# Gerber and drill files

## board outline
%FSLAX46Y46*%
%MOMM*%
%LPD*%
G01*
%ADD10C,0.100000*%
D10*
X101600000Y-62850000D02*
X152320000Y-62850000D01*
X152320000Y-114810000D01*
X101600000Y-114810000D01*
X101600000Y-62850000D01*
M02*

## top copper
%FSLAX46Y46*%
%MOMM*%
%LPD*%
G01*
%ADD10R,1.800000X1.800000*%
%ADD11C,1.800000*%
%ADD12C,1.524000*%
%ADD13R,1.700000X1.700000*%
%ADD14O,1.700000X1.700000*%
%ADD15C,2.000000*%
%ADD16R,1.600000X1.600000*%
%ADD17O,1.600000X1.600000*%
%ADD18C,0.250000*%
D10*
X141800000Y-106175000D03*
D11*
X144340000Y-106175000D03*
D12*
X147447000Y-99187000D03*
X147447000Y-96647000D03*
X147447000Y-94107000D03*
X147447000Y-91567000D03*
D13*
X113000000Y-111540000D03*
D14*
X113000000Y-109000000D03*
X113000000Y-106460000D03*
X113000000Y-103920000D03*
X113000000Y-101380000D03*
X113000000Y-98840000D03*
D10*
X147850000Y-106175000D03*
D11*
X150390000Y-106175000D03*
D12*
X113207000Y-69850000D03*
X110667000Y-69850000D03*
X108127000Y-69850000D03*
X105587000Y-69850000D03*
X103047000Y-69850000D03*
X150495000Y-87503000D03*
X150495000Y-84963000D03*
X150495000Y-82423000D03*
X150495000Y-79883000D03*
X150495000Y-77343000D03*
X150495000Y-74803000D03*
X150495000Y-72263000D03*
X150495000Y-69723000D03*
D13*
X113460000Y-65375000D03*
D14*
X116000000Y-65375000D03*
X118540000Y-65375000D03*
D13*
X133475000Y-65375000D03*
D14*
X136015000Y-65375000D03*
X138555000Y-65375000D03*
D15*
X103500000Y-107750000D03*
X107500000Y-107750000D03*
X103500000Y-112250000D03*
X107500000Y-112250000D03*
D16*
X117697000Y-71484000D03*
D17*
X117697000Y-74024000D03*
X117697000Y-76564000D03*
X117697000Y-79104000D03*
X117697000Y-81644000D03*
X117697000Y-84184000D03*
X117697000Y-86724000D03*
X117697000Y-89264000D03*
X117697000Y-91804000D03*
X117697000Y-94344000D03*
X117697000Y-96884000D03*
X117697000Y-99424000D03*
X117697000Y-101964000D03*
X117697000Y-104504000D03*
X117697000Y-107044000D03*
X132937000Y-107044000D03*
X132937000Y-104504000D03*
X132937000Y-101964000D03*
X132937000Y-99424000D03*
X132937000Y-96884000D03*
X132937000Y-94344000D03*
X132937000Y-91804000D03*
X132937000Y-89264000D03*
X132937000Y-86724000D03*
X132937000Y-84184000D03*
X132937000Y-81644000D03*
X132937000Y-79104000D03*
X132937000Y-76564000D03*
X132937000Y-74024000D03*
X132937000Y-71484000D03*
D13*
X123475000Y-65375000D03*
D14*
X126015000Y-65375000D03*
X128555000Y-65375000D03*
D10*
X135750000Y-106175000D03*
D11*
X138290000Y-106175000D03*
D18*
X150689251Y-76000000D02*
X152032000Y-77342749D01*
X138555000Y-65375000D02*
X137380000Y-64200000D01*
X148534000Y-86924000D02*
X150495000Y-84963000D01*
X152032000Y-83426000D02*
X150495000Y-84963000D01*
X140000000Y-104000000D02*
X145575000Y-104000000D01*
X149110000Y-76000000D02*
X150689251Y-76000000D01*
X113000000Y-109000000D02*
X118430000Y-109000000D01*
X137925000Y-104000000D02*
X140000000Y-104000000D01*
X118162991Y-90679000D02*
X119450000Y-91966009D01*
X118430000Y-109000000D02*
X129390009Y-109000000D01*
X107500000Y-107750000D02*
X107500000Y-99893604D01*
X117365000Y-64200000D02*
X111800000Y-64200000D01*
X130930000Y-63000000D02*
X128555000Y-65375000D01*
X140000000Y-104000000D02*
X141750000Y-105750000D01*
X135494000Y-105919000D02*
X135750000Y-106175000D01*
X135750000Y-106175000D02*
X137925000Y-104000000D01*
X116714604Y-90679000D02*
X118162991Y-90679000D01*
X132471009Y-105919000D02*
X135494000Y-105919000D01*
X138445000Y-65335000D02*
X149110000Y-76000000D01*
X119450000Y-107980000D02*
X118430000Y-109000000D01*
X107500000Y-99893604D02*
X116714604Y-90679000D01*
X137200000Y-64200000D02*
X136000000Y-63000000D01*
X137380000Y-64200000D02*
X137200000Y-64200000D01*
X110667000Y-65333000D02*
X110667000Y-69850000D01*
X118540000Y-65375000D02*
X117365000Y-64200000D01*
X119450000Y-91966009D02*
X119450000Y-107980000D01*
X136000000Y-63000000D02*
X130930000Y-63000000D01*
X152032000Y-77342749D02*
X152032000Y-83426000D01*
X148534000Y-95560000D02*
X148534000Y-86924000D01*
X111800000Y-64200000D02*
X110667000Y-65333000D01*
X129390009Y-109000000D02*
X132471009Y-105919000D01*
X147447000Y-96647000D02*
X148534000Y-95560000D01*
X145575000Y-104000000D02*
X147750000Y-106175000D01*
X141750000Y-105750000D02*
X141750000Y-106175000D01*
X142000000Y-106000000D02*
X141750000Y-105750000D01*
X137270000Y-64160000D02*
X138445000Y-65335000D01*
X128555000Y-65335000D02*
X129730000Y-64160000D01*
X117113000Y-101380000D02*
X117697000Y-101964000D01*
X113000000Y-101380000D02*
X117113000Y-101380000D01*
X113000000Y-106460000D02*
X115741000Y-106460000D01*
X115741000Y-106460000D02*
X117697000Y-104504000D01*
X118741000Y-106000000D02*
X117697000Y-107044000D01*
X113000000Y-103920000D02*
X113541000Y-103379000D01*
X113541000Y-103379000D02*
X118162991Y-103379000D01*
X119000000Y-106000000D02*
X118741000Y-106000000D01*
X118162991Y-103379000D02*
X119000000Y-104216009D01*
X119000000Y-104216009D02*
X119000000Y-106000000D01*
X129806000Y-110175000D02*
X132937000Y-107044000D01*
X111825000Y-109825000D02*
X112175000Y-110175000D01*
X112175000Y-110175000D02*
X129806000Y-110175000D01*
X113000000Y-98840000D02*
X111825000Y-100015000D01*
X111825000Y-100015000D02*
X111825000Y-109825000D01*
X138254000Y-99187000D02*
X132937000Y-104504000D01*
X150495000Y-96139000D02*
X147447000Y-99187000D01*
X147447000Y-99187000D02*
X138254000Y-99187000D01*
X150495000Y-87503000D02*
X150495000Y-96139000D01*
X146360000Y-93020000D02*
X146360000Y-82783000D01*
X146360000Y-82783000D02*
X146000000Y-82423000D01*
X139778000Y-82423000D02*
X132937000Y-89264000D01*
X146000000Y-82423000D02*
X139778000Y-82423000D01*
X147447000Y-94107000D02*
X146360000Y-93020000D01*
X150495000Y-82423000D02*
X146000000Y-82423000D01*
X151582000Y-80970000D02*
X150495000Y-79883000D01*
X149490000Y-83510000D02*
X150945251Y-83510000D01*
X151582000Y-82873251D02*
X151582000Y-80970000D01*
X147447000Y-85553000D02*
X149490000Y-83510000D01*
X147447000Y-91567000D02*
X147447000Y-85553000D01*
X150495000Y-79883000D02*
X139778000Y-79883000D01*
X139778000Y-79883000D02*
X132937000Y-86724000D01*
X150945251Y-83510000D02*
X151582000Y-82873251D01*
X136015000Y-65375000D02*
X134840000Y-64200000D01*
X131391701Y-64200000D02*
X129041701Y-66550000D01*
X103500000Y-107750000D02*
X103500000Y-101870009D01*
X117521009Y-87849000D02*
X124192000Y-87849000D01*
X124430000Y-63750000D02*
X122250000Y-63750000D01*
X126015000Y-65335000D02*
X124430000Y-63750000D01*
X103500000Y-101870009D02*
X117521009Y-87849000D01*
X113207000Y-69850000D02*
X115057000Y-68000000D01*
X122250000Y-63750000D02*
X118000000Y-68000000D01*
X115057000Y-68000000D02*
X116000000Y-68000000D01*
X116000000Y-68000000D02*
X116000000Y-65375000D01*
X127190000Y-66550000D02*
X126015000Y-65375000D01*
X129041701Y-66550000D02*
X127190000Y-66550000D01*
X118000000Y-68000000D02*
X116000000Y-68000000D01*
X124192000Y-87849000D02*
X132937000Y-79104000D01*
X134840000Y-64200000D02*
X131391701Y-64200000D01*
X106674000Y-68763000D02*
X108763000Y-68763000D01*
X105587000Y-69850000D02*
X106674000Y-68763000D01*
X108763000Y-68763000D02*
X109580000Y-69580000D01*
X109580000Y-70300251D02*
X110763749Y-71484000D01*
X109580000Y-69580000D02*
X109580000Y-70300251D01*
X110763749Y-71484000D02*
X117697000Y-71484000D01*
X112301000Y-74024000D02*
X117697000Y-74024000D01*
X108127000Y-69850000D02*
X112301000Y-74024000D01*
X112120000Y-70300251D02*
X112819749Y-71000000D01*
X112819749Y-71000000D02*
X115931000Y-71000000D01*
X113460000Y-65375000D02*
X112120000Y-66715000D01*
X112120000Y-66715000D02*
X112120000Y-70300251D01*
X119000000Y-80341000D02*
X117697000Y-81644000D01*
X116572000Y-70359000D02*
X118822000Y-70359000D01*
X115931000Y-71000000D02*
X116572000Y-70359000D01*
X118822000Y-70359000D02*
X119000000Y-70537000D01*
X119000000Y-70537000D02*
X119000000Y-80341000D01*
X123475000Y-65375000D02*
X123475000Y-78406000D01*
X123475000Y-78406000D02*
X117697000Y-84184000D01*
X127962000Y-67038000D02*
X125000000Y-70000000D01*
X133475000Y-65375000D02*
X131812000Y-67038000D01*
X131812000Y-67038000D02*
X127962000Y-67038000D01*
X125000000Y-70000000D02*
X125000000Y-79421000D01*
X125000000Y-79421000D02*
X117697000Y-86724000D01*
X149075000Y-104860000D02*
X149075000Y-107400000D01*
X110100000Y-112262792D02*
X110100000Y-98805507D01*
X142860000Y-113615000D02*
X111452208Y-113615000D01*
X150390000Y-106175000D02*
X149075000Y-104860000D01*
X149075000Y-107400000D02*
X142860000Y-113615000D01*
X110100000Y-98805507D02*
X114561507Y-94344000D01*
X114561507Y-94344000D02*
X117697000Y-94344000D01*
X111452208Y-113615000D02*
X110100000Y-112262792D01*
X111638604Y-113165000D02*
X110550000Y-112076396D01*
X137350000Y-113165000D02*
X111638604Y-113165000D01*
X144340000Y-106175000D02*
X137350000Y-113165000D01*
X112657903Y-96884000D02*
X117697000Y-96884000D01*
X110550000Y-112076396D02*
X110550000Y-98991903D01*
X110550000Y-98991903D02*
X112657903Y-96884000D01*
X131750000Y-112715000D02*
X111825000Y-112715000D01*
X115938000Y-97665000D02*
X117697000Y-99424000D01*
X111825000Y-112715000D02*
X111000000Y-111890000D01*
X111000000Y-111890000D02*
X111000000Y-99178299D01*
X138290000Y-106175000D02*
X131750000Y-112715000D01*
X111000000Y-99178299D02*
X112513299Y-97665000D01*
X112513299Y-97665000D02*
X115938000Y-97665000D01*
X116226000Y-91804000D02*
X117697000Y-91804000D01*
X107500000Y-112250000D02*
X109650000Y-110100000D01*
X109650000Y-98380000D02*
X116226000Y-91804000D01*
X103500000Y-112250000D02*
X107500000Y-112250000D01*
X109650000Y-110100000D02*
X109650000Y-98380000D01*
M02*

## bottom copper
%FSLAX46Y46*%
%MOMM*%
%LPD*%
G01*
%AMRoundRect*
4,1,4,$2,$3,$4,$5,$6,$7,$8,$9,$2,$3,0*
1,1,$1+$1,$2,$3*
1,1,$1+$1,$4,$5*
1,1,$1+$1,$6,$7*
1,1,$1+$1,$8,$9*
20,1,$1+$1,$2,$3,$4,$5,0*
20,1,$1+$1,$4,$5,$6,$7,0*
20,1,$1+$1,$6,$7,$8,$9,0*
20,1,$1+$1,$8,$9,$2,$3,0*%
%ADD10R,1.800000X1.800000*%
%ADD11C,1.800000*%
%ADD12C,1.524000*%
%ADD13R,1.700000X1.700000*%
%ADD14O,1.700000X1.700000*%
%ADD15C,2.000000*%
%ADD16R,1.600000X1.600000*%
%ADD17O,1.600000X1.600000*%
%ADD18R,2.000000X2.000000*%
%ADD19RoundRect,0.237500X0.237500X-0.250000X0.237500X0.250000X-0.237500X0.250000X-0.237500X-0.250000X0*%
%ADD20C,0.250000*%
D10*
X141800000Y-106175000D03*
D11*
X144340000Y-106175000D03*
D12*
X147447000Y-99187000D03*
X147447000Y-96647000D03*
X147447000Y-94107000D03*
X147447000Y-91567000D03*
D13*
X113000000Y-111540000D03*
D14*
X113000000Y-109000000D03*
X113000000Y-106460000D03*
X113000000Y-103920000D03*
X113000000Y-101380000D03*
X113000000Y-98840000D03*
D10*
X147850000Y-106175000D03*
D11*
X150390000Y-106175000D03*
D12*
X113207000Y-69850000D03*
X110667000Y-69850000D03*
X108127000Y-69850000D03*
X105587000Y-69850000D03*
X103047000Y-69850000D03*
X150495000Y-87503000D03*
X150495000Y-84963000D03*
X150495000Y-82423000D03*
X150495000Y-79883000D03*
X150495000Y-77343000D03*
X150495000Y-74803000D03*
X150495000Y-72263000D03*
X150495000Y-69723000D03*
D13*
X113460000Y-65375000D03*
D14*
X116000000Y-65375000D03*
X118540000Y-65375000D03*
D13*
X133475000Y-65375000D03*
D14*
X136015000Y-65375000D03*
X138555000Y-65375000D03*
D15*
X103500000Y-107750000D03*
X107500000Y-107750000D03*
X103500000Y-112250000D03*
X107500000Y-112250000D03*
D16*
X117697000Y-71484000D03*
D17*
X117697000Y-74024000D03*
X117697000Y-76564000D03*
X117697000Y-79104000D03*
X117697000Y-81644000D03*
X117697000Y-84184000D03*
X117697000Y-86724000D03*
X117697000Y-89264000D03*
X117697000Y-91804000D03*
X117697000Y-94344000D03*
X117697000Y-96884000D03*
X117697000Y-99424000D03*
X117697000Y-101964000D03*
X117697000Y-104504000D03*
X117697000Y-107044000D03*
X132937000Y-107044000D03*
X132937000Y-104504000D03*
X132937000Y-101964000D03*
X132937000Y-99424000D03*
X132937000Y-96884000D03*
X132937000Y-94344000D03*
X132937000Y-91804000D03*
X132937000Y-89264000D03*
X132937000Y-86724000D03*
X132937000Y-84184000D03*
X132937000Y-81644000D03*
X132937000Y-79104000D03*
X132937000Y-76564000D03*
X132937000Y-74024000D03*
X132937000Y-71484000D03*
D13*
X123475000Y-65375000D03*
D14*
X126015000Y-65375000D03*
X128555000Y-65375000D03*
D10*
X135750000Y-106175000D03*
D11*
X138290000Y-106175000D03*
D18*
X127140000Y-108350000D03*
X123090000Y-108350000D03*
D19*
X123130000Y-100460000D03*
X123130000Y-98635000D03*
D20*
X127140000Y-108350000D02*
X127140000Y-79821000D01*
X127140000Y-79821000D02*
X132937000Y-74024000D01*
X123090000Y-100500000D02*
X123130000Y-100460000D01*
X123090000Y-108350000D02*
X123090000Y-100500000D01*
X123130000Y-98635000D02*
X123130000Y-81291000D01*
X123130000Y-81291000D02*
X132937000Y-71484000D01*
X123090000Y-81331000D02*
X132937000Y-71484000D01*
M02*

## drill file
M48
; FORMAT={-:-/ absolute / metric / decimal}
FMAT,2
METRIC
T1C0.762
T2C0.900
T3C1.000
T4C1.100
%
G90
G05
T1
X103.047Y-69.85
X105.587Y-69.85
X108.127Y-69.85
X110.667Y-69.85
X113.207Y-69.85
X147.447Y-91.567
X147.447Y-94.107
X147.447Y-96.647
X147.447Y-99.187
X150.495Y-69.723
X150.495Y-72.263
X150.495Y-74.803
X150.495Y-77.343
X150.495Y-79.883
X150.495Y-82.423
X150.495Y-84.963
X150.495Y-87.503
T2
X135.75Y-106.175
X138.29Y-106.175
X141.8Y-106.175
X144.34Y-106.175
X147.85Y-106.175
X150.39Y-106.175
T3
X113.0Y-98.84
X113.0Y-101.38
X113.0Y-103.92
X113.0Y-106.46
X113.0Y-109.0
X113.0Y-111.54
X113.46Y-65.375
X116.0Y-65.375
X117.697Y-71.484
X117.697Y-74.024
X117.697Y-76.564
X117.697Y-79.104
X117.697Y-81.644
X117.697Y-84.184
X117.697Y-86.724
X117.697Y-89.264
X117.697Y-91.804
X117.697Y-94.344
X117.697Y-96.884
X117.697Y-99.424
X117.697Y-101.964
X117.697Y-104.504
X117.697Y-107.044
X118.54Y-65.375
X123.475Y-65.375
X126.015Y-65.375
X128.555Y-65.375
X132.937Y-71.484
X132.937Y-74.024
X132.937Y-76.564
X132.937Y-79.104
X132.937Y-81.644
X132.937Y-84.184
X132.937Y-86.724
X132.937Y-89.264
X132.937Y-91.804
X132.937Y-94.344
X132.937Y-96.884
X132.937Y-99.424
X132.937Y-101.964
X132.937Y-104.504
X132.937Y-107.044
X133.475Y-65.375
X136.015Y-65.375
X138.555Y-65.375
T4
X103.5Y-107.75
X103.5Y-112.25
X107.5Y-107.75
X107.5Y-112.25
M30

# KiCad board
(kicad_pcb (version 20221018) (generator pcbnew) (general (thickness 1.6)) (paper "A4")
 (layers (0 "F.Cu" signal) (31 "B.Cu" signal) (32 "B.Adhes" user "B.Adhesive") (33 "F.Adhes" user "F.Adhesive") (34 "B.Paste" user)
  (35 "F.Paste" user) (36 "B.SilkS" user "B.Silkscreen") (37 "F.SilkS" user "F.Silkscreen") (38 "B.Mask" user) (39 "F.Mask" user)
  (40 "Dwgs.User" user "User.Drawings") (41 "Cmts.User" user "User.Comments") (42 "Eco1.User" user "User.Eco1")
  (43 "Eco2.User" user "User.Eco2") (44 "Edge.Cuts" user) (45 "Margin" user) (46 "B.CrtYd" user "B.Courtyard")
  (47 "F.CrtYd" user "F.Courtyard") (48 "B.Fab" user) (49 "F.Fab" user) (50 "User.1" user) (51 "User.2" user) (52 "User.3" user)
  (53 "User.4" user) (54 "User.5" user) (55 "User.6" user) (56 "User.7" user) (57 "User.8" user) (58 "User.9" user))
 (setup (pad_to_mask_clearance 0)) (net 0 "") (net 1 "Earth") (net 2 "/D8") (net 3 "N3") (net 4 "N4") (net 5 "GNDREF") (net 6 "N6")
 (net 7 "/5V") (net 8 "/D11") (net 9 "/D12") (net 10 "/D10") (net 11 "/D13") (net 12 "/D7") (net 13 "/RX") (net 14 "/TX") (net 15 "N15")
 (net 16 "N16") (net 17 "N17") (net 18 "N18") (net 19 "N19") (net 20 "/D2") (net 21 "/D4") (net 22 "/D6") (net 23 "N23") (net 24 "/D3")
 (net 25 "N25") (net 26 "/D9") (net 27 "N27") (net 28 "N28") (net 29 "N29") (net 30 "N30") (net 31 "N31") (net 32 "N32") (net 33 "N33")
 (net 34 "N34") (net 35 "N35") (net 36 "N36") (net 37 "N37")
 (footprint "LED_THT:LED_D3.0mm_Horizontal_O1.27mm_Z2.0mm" (layer "F.Cu") (at 141.8 106.175)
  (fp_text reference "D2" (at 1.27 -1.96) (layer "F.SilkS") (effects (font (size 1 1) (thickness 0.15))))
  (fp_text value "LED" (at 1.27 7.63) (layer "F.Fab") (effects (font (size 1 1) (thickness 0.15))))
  (pad "1" thru_hole rect (at 0 0) (size 1.8 1.8) (drill 0.9) (layers "*.Cu" "*.Mask") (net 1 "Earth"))
  (pad "2" thru_hole circle (at 2.54 0) (size 1.8 1.8) (drill 0.9) (layers "*.Cu" "*.Mask") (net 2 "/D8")))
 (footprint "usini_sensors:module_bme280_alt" (layer "F.Cu") (at 147.447 91.567 180)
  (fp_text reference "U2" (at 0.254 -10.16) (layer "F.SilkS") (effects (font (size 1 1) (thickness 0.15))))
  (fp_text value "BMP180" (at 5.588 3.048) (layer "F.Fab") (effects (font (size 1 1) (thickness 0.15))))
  (pad "1" thru_hole circle (at 0 -7.62 180) (size 1.524 1.524) (drill 0.762) (layers "*.Cu" "*.Mask") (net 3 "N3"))
  (pad "2" thru_hole circle (at 0 -5.08 180) (size 1.524 1.524) (drill 0.762) (layers "*.Cu" "*.Mask") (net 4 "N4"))
  (pad "3" thru_hole circle (at 0 -2.54 180) (size 1.524 1.524) (drill 0.762) (layers "*.Cu" "*.Mask") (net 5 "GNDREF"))
  (pad "4" thru_hole circle (at 0 0 180) (size 1.524 1.524) (drill 0.762) (layers "*.Cu" "*.Mask") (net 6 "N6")))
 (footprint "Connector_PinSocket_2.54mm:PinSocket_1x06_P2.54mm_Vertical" (layer "F.Cu") (at 113 111.54 180)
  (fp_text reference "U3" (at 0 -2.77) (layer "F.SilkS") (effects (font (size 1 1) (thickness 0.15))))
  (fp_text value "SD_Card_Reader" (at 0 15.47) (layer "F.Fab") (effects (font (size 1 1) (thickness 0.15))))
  (pad "1" thru_hole rect (at 0 0 180) (size 1.7 1.7) (drill 1) (layers "*.Cu" "*.Mask") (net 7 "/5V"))
  (pad "2" thru_hole oval (at 0 2.54 180) (size 1.7 1.7) (drill 1) (layers "*.Cu" "*.Mask") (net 1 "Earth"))
  (pad "3" thru_hole oval (at 0 5.08 180) (size 1.7 1.7) (drill 1) (layers "*.Cu" "*.Mask") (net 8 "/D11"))
  (pad "4" thru_hole oval (at 0 7.62 180) (size 1.7 1.7) (drill 1) (layers "*.Cu" "*.Mask") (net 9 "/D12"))
  (pad "5" thru_hole oval (at 0 10.16 180) (size 1.7 1.7) (drill 1) (layers "*.Cu" "*.Mask") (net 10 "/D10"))
  (pad "6" thru_hole oval (at 0 12.7 180) (size 1.7 1.7) (drill 1) (layers "*.Cu" "*.Mask") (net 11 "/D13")))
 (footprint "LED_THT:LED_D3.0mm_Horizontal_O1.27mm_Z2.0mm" (layer "F.Cu") (at 147.85 106.175)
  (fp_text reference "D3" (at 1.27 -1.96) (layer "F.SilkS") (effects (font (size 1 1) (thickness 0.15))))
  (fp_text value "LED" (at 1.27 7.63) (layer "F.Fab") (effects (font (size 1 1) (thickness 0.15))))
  (pad "1" thru_hole rect (at 0 0) (size 1.8 1.8) (drill 0.9) (layers "*.Cu" "*.Mask") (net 1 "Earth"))
  (pad "2" thru_hole circle (at 2.54 0) (size 1.8 1.8) (drill 0.9) (layers "*.Cu" "*.Mask") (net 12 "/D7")))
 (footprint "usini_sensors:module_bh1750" (layer "F.Cu") (at 103.047 69.85 -90)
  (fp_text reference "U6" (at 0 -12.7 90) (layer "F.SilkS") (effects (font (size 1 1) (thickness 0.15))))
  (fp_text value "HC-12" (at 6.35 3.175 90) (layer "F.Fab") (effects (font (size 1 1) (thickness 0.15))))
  (pad "1" thru_hole circle (at 0 -10.16 270) (size 1.524 1.524) (drill 0.762) (layers "*.Cu" "*.Mask") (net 6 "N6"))
  (pad "2" thru_hole circle (at 0 -7.62 270) (size 1.524 1.524) (drill 0.762) (layers "*.Cu" "*.Mask") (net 5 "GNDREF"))
  (pad "3" thru_hole circle (at 0 -5.08 270) (size 1.524 1.524) (drill 0.762) (layers "*.Cu" "*.Mask") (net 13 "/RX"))
  (pad "4" thru_hole circle (at 0 -2.54 270) (size 1.524 1.524) (drill 0.762) (layers "*.Cu" "*.Mask") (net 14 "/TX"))
  (pad "5" thru_hole circle (at 0 0 270) (size 1.524 1.524) (drill 0.762) (layers "*.Cu" "*.Mask") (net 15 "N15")))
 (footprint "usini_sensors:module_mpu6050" (layer "F.Cu") (at 150.495 69.723 180)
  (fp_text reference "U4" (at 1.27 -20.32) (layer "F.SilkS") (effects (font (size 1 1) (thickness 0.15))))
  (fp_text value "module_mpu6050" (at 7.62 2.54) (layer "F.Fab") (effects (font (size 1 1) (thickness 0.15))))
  (pad "1" thru_hole circle (at 0 -17.78 180) (size 1.524 1.524) (drill 0.762) (layers "*.Cu" "*.Mask") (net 6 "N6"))
  (pad "2" thru_hole circle (at 0 -15.24 180) (size 1.524 1.524) (drill 0.762) (layers "*.Cu" "*.Mask") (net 5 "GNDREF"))
  (pad "3" thru_hole circle (at 0 -12.7 180) (size 1.524 1.524) (drill 0.762) (layers "*.Cu" "*.Mask") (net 4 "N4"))
  (pad "4" thru_hole circle (at 0 -10.16 180) (size 1.524 1.524) (drill 0.762) (layers "*.Cu" "*.Mask") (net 3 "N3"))
  (pad "5" thru_hole circle (at 0 -7.62 180) (size 1.524 1.524) (drill 0.762) (layers "*.Cu" "*.Mask") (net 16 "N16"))
  (pad "6" thru_hole circle (at 0 -5.08 180) (size 1.524 1.524) (drill 0.762) (layers "*.Cu" "*.Mask") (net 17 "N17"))
  (pad "7" thru_hole circle (at 0 -2.54 180) (size 1.524 1.524) (drill 0.762) (layers "*.Cu" "*.Mask") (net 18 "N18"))
  (pad "8" thru_hole circle (at 0 0 180) (size 1.524 1.524) (drill 0.762) (layers "*.Cu" "*.Mask") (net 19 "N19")))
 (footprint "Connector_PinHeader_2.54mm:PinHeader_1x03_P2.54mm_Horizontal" (layer "F.Cu") (at 113.46 65.375 90)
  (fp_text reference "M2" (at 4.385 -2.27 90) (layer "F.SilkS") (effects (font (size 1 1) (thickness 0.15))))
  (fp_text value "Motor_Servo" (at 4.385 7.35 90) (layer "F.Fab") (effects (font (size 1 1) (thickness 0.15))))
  (pad "1" thru_hole rect (at 0 0 90) (size 1.7 1.7) (drill 1) (layers "*.Cu" "*.Mask") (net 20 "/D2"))
  (pad "2" thru_hole oval (at 0 2.54 90) (size 1.7 1.7) (drill 1) (layers "*.Cu" "*.Mask") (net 7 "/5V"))
  (pad "3" thru_hole oval (at 0 5.08 90) (size 1.7 1.7) (drill 1) (layers "*.Cu" "*.Mask") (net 1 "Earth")))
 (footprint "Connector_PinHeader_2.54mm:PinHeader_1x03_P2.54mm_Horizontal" (layer "F.Cu") (at 133.475 65.375 90)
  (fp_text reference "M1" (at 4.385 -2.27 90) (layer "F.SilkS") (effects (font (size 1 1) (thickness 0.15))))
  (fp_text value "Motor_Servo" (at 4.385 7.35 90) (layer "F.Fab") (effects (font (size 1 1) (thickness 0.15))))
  (pad "1" thru_hole rect (at 0 0 90) (size 1.7 1.7) (drill 1) (layers "*.Cu" "*.Mask") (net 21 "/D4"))
  (pad "2" thru_hole oval (at 0 2.54 90) (size 1.7 1.7) (drill 1) (layers "*.Cu" "*.Mask") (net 7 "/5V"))
  (pad "3" thru_hole oval (at 0 5.08 90) (size 1.7 1.7) (drill 1) (layers "*.Cu" "*.Mask") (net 1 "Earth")))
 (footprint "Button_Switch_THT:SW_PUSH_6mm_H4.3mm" (layer "F.Cu") (at 101 107.75)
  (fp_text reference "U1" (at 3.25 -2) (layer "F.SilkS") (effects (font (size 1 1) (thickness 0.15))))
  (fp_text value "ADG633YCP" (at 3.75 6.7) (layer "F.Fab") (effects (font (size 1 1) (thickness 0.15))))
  (pad "1" thru_hole circle (at 2.5 0 90) (size 2 2) (drill 1.1) (layers "*.Cu" "*.Mask") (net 7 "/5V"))
  (pad "1" thru_hole circle (at 6.5 0 90) (size 2 2) (drill 1.1) (layers "*.Cu" "*.Mask") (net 7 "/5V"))
  (pad "2" thru_hole circle (at 2.5 4.5 90) (size 2 2) (drill 1.1) (layers "*.Cu" "*.Mask") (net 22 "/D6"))
  (pad "2" thru_hole circle (at 6.5 4.5 90) (size 2 2) (drill 1.1) (layers "*.Cu" "*.Mask") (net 22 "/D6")))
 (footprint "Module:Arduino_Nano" (layer "F.Cu") (at 117.697 71.484)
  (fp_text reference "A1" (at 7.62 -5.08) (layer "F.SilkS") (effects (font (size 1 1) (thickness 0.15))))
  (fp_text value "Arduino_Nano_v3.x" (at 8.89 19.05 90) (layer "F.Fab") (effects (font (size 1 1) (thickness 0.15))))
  (pad "1" thru_hole rect (at 0 0) (size 1.6 1.6) (drill 1) (layers "*.Cu" "*.Mask") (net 14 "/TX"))
  (pad "2" thru_hole oval (at 0 2.54) (size 1.6 1.6) (drill 1) (layers "*.Cu" "*.Mask") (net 13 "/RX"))
  (pad "3" thru_hole oval (at 0 5.08) (size 1.6 1.6) (drill 1) (layers "*.Cu" "*.Mask") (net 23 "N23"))
  (pad "4" thru_hole oval (at 0 7.62) (size 1.6 1.6) (drill 1) (layers "*.Cu" "*.Mask") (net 1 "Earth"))
  (pad "5" thru_hole oval (at 0 10.16) (size 1.6 1.6) (drill 1) (layers "*.Cu" "*.Mask") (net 20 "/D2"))
  (pad "6" thru_hole oval (at 0 12.7) (size 1.6 1.6) (drill 1) (layers "*.Cu" "*.Mask") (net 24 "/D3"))
  (pad "7" thru_hole oval (at 0 15.24) (size 1.6 1.6) (drill 1) (layers "*.Cu" "*.Mask") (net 21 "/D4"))
  (pad "8" thru_hole oval (at 0 17.78) (size 1.6 1.6) (drill 1) (layers "*.Cu" "*.Mask") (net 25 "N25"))
  (pad "9" thru_hole oval (at 0 20.32) (size 1.6 1.6) (drill 1) (layers "*.Cu" "*.Mask") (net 22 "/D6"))
  (pad "10" thru_hole oval (at 0 22.86) (size 1.6 1.6) (drill 1) (layers "*.Cu" "*.Mask") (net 12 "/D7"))
  (pad "11" thru_hole oval (at 0 25.4) (size 1.6 1.6) (drill 1) (layers "*.Cu" "*.Mask") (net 2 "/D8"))
  (pad "12" thru_hole oval (at 0 27.94) (size 1.6 1.6) (drill 1) (layers "*.Cu" "*.Mask") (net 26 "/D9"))
  (pad "13" thru_hole oval (at 0 30.48) (size 1.6 1.6) (drill 1) (layers "*.Cu" "*.Mask") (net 10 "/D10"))
  (pad "14" thru_hole oval (at 0 33.02) (size 1.6 1.6) (drill 1) (layers "*.Cu" "*.Mask") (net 8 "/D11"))
  (pad "15" thru_hole oval (at 0 35.56) (size 1.6 1.6) (drill 1) (layers "*.Cu" "*.Mask") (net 9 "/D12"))
  (pad "16" thru_hole oval (at 15.24 35.56) (size 1.6 1.6) (drill 1) (layers "*.Cu" "*.Mask") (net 11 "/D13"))
  (pad "17" thru_hole oval (at 15.24 33.02) (size 1.6 1.6) (drill 1) (layers "*.Cu" "*.Mask") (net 6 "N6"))
  (pad "18" thru_hole oval (at 15.24 30.48) (size 1.6 1.6) (drill 1) (layers "*.Cu" "*.Mask") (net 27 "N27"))
  (pad "19" thru_hole oval (at 15.24 27.94) (size 1.6 1.6) (drill 1) (layers "*.Cu" "*.Mask") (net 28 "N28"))
  (pad "20" thru_hole oval (at 15.24 25.4) (size 1.6 1.6) (drill 1) (layers "*.Cu" "*.Mask") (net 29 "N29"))
  (pad "21" thru_hole oval (at 15.24 22.86) (size 1.6 1.6) (drill 1) (layers "*.Cu" "*.Mask") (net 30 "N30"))
  (pad "22" thru_hole oval (at 15.24 20.32) (size 1.6 1.6) (drill 1) (layers "*.Cu" "*.Mask") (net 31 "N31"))
  (pad "23" thru_hole oval (at 15.24 17.78) (size 1.6 1.6) (drill 1) (layers "*.Cu" "*.Mask") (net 4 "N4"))
  (pad "24" thru_hole oval (at 15.24 15.24) (size 1.6 1.6) (drill 1) (layers "*.Cu" "*.Mask") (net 3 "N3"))
  (pad "25" thru_hole oval (at 15.24 12.7) (size 1.6 1.6) (drill 1) (layers "*.Cu" "*.Mask") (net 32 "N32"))
  (pad "26" thru_hole oval (at 15.24 10.16) (size 1.6 1.6) (drill 1) (layers "*.Cu" "*.Mask") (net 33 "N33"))
  (pad "27" thru_hole oval (at 15.24 7.62) (size 1.6 1.6) (drill 1) (layers "*.Cu" "*.Mask") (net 7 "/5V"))
  (pad "28" thru_hole oval (at 15.24 5.08) (size 1.6 1.6) (drill 1) (layers "*.Cu" "*.Mask") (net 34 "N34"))
  (pad "29" thru_hole oval (at 15.24 2.54) (size 1.6 1.6) (drill 1) (layers "*.Cu" "*.Mask") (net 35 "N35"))
  (pad "30" thru_hole oval (at 15.24 0) (size 1.6 1.6) (drill 1) (layers "*.Cu" "*.Mask") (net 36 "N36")))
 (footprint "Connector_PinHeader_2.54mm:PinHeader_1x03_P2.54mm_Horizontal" (layer "F.Cu") (at 123.475 65.375 90)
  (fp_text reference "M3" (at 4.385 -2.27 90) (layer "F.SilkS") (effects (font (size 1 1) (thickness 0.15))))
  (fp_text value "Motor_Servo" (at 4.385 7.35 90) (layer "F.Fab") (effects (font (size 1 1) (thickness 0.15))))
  (pad "1" thru_hole rect (at 0 0 90) (size 1.7 1.7) (drill 1) (layers "*.Cu" "*.Mask") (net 24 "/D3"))
  (pad "2" thru_hole oval (at 0 2.54 90) (size 1.7 1.7) (drill 1) (layers "*.Cu" "*.Mask") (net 7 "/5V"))
  (pad "3" thru_hole oval (at 0 5.08 90) (size 1.7 1.7) (drill 1) (layers "*.Cu" "*.Mask") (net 1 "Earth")))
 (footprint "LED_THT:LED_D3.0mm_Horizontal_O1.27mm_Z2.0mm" (layer "F.Cu") (at 135.75 106.175)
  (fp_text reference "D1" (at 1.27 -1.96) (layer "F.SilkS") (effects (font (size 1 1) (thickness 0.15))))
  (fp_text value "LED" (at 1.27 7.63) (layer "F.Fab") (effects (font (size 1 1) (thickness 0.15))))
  (pad "1" thru_hole rect (at 0 0) (size 1.8 1.8) (drill 0.9) (layers "*.Cu" "*.Mask") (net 1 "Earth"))
  (pad "2" thru_hole circle (at 2.54 0) (size 1.8 1.8) (drill 0.9) (layers "*.Cu" "*.Mask") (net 26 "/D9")))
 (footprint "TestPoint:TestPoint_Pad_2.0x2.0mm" (layer "B.Cu") (at 127.14 108.35 -90)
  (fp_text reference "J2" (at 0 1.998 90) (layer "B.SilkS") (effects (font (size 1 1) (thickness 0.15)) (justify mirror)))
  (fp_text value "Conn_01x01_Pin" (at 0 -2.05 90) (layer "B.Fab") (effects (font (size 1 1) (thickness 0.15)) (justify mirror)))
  (pad "1" smd rect (at 0 0 270) (size 2 2) (layers "B.Cu" "B.Mask") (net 35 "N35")))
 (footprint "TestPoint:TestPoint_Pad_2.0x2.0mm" (layer "B.Cu") (at 123.09 108.35 -90)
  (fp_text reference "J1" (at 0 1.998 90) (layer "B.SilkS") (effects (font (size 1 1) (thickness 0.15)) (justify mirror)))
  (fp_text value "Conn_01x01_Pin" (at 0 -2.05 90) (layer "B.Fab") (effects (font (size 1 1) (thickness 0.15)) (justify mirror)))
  (pad "1" smd rect (at 0 0 270) (size 2 2) (layers "B.Cu" "B.Mask") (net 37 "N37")))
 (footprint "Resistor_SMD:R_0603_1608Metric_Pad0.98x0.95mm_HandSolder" (layer "B.Cu") (at 123.13 99.5475 90)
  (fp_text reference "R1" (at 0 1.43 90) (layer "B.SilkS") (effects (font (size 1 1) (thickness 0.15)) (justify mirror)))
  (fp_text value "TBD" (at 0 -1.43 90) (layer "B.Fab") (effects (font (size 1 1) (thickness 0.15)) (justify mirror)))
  (pad "1" smd roundrect (at -0.9125 0 90) (size 0.975 0.95) (layers "B.Cu" "B.Paste" "B.Mask") (roundrect_rratio 0.25) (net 37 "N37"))
  (pad "2" smd roundrect (at 0.9125 0 90) (size 0.975 0.95) (layers "B.Cu" "B.Paste" "B.Mask") (roundrect_rratio 0.25) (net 36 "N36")))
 (gr_rect (start 101.6 62.85) (end 152.32 114.81) (stroke (width 0.1) (type default)) (fill none) (layer "Edge.Cuts"))
 (segment (start 150.689251 76) (end 152.032 77.342749) (width 0.25) (layer "F.Cu") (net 1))
 (segment (start 138.555 65.375) (end 137.38 64.2) (width 0.25) (layer "F.Cu") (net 1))
 (segment (start 148.534 86.924) (end 150.495 84.963) (width 0.25) (layer "F.Cu") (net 1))
 (segment (start 152.032 83.426) (end 150.495 84.963) (width 0.25) (layer "F.Cu") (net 1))
 (segment (start 140 104) (end 145.575 104) (width 0.25) (layer "F.Cu") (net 1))
 (segment (start 149.11 76) (end 150.689251 76) (width 0.25) (layer "F.Cu") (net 1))
 (segment (start 113 109) (end 118.43 109) (width 0.25) (layer "F.Cu") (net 1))
 (segment (start 137.925 104) (end 140 104) (width 0.25) (layer "F.Cu") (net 1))
 (segment (start 118.162991 90.679) (end 119.45 91.966009) (width 0.25) (layer "F.Cu") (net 1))
 (segment (start 118.43 109) (end 129.390009 109) (width 0.25) (layer "F.Cu") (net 1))
 (segment (start 107.5 107.75) (end 107.5 99.893604) (width 0.25) (layer "F.Cu") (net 1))
 (segment (start 117.365 64.2) (end 111.8 64.2) (width 0.25) (layer "F.Cu") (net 1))
 (segment (start 130.93 63) (end 128.555 65.375) (width 0.25) (layer "F.Cu") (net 1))
 (segment (start 140 104) (end 141.75 105.75) (width 0.25) (layer "F.Cu") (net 1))
 (segment (start 135.494 105.919) (end 135.75 106.175) (width 0.25) (layer "F.Cu") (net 1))
 (segment (start 135.75 106.175) (end 137.925 104) (width 0.25) (layer "F.Cu") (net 1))
 (segment (start 116.714604 90.679) (end 118.162991 90.679) (width 0.25) (layer "F.Cu") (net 1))
 (segment (start 132.471009 105.919) (end 135.494 105.919) (width 0.25) (layer "F.Cu") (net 1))
 (segment (start 138.445 65.335) (end 149.11 76) (width 0.25) (layer "F.Cu") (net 1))
 (segment (start 119.45 107.98) (end 118.43 109) (width 0.25) (layer "F.Cu") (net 1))
 (segment (start 107.5 99.893604) (end 116.714604 90.679) (width 0.25) (layer "F.Cu") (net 1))
 (segment (start 137.2 64.2) (end 136 63) (width 0.25) (layer "F.Cu") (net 1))
 (segment (start 137.38 64.2) (end 137.2 64.2) (width 0.25) (layer "F.Cu") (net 1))
 (segment (start 110.667 65.333) (end 110.667 69.85) (width 0.25) (layer "F.Cu") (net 1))
 (segment (start 118.54 65.375) (end 117.365 64.2) (width 0.25) (layer "F.Cu") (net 1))
 (segment (start 119.45 91.966009) (end 119.45 107.98) (width 0.25) (layer "F.Cu") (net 1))
 (segment (start 136 63) (end 130.93 63) (width 0.25) (layer "F.Cu") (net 1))
 (segment (start 152.032 77.342749) (end 152.032 83.426) (width 0.25) (layer "F.Cu") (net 1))
 (segment (start 148.534 95.56) (end 148.534 86.924) (width 0.25) (layer "F.Cu") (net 1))
 (segment (start 111.8 64.2) (end 110.667 65.333) (width 0.25) (layer "F.Cu") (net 1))
 (segment (start 129.390009 109) (end 132.471009 105.919) (width 0.25) (layer "F.Cu") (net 1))
 (segment (start 147.447 96.647) (end 148.534 95.56) (width 0.25) (layer "F.Cu") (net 1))
 (segment (start 145.575 104) (end 147.75 106.175) (width 0.25) (layer "F.Cu") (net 1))
 (segment (start 141.75 105.75) (end 141.75 106.175) (width 0.25) (layer "F.Cu") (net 1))
 (segment (start 142 106) (end 141.75 105.75) (width 0.25) (layer "F.Cu") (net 1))
 (segment (start 137.27 64.16) (end 138.445 65.335) (width 0.25) (layer "F.Cu") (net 1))
 (segment (start 128.555 65.335) (end 129.73 64.16) (width 0.25) (layer "F.Cu") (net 1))
 (segment (start 117.113 101.38) (end 117.697 101.964) (width 0.25) (layer "F.Cu") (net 10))
 (segment (start 113 101.38) (end 117.113 101.38) (width 0.25) (layer "F.Cu") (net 10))
 (segment (start 113 106.46) (end 115.741 106.46) (width 0.25) (layer "F.Cu") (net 8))
 (segment (start 115.741 106.46) (end 117.697 104.504) (width 0.25) (layer "F.Cu") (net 8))
 (segment (start 118.741 106) (end 117.697 107.044) (width 0.25) (layer "F.Cu") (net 9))
 (segment (start 113 103.92) (end 113.541 103.379) (width 0.25) (layer "F.Cu") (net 9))
 (segment (start 113.541 103.379) (end 118.162991 103.379) (width 0.25) (layer "F.Cu") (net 9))
 (segment (start 119 106) (end 118.741 106) (width 0.25) (layer "F.Cu") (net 9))
 (segment (start 118.162991 103.379) (end 119 104.216009) (width 0.25) (layer "F.Cu") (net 9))
 (segment (start 119 104.216009) (end 119 106) (width 0.25) (layer "F.Cu") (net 9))
 (segment (start 129.806 110.175) (end 132.937 107.044) (width 0.25) (layer "F.Cu") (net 11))
 (segment (start 111.825 109.825) (end 112.175 110.175) (width 0.25) (layer "F.Cu") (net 11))
 (segment (start 112.175 110.175) (end 129.806 110.175) (width 0.25) (layer "F.Cu") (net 11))
 (segment (start 113 98.84) (end 111.825 100.015) (width 0.25) (layer "F.Cu") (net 11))
 (segment (start 111.825 100.015) (end 111.825 109.825) (width 0.25) (layer "F.Cu") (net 11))
 (segment (start 138.254 99.187) (end 132.937 104.504) (width 0.25) (layer "F.Cu") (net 6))
 (segment (start 150.495 96.139) (end 147.447 99.187) (width 0.25) (layer "F.Cu") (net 6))
 (segment (start 147.447 99.187) (end 138.254 99.187) (width 0.25) (layer "F.Cu") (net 6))
 (segment (start 150.495 87.503) (end 150.495 96.139) (width 0.25) (layer "F.Cu") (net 6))
 (segment (start 146.36 93.02) (end 146.36 82.783) (width 0.25) (layer "F.Cu") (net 4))
 (segment (start 146.36 82.783) (end 146 82.423) (width 0.25) (layer "F.Cu") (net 4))
 (segment (start 139.778 82.423) (end 132.937 89.264) (width 0.25) (layer "F.Cu") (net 4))
 (segment (start 146 82.423) (end 139.778 82.423) (width 0.25) (layer "F.Cu") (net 4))
 (segment (start 147.447 94.107) (end 146.36 93.02) (width 0.25) (layer "F.Cu") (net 4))
 (segment (start 150.495 82.423) (end 146 82.423) (width 0.25) (layer "F.Cu") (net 4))
 (segment (start 151.582 80.97) (end 150.495 79.883) (width 0.25) (layer "F.Cu") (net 3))
 (segment (start 149.49 83.51) (end 150.945251 83.51) (width 0.25) (layer "F.Cu") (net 3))
 (segment (start 151.582 82.873251) (end 151.582 80.97) (width 0.25) (layer "F.Cu") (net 3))
 (segment (start 147.447 85.553) (end 149.49 83.51) (width 0.25) (layer "F.Cu") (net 3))
 (segment (start 147.447 91.567) (end 147.447 85.553) (width 0.25) (layer "F.Cu") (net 3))
 (segment (start 150.495 79.883) (end 139.778 79.883) (width 0.25) (layer "F.Cu") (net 3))
 (segment (start 139.778 79.883) (end 132.937 86.724) (width 0.25) (layer "F.Cu") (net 3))
 (segment (start 150.945251 83.51) (end 151.582 82.873251) (width 0.25) (layer "F.Cu") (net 3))
 (segment (start 136.015 65.375) (end 134.84 64.2) (width 0.25) (layer "F.Cu") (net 7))
 (segment (start 131.391701 64.2) (end 129.041701 66.55) (width 0.25) (layer "F.Cu") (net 7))
 (segment (start 103.5 107.75) (end 103.5 101.870009) (width 0.25) (layer "F.Cu") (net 7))
 (segment (start 117.521009 87.849) (end 124.192 87.849) (width 0.25) (layer "F.Cu") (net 7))
 (segment (start 124.43 63.75) (end 122.25 63.75) (width 0.25) (layer "F.Cu") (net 7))
 (segment (start 126.015 65.335) (end 124.43 63.75) (width 0.25) (layer "F.Cu") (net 7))
 (segment (start 103.5 101.870009) (end 117.521009 87.849) (width 0.25) (layer "F.Cu") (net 7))
 (segment (start 113.207 69.85) (end 115.057 68) (width 0.25) (layer "F.Cu") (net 7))
 (segment (start 122.25 63.75) (end 118 68) (width 0.25) (layer "F.Cu") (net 7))
 (segment (start 115.057 68) (end 116 68) (width 0.25) (layer "F.Cu") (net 7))
 (segment (start 116 68) (end 116 65.375) (width 0.25) (layer "F.Cu") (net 7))
 (segment (start 127.19 66.55) (end 126.015 65.375) (width 0.25) (layer "F.Cu") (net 7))
 (segment (start 129.041701 66.55) (end 127.19 66.55) (width 0.25) (layer "F.Cu") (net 7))
 (segment (start 118 68) (end 116 68) (width 0.25) (layer "F.Cu") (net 7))
 (segment (start 124.192 87.849) (end 132.937 79.104) (width 0.25) (layer "F.Cu") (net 7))
 (segment (start 134.84 64.2) (end 131.391701 64.2) (width 0.25) (layer "F.Cu") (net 7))
 (segment (start 106.674 68.763) (end 108.763 68.763) (width 0.25) (layer "F.Cu") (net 14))
 (segment (start 105.587 69.85) (end 106.674 68.763) (width 0.25) (layer "F.Cu") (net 14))
 (segment (start 108.763 68.763) (end 109.58 69.58) (width 0.25) (layer "F.Cu") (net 14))
 (segment (start 109.58 70.300251) (end 110.763749 71.484) (width 0.25) (layer "F.Cu") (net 14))
 (segment (start 109.58 69.58) (end 109.58 70.300251) (width 0.25) (layer "F.Cu") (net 14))
 (segment (start 110.763749 71.484) (end 117.697 71.484) (width 0.25) (layer "F.Cu") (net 14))
 (segment (start 112.301 74.024) (end 117.697 74.024) (width 0.25) (layer "F.Cu") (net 13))
 (segment (start 108.127 69.85) (end 112.301 74.024) (width 0.25) (layer "F.Cu") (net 13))
 (segment (start 112.12 70.300251) (end 112.819749 71) (width 0.25) (layer "F.Cu") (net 20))
 (segment (start 112.819749 71) (end 115.931 71) (width 0.25) (layer "F.Cu") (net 20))
 (segment (start 113.46 65.375) (end 112.12 66.715) (width 0.25) (layer "F.Cu") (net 20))
 (segment (start 112.12 66.715) (end 112.12 70.300251) (width 0.25) (layer "F.Cu") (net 20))
 (segment (start 119 80.341) (end 117.697 81.644) (width 0.25) (layer "F.Cu") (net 20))
 (segment (start 116.572 70.359) (end 118.822 70.359) (width 0.25) (layer "F.Cu") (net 20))
 (segment (start 115.931 71) (end 116.572 70.359) (width 0.25) (layer "F.Cu") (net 20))
 (segment (start 118.822 70.359) (end 119 70.537) (width 0.25) (layer "F.Cu") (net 20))
 (segment (start 119 70.537) (end 119 80.341) (width 0.25) (layer "F.Cu") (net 20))
 (segment (start 123.475 65.375) (end 123.475 78.406) (width 0.25) (layer "F.Cu") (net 24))
 (segment (start 123.475 78.406) (end 117.697 84.184) (width 0.25) (layer "F.Cu") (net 24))
 (segment (start 127.962 67.038) (end 125 70) (width 0.25) (layer "F.Cu") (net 21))
 (segment (start 133.475 65.375) (end 131.812 67.038) (width 0.25) (layer "F.Cu") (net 21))
 (segment (start 131.812 67.038) (end 127.962 67.038) (width 0.25) (layer "F.Cu") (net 21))
 (segment (start 125 70) (end 125 79.421) (width 0.25) (layer "F.Cu") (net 21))
 (segment (start 125 79.421) (end 117.697 86.724) (width 0.25) (layer "F.Cu") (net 21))
 (segment (start 149.075 104.86) (end 149.075 107.4) (width 0.25) (layer "F.Cu") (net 12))
 (segment (start 110.1 112.262792) (end 110.1 98.805507) (width 0.25) (layer "F.Cu") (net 12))
 (segment (start 142.86 113.615) (end 111.452208 113.615) (width 0.25) (layer "F.Cu") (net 12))
 (segment (start 150.39 106.175) (end 149.075 104.86) (width 0.25) (layer "F.Cu") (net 12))
 (segment (start 149.075 107.4) (end 142.86 113.615) (width 0.25) (layer "F.Cu") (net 12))
 (segment (start 110.1 98.805507) (end 114.561507 94.344) (width 0.25) (layer "F.Cu") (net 12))
 (segment (start 114.561507 94.344) (end 117.697 94.344) (width 0.25) (layer "F.Cu") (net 12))
 (segment (start 111.452208 113.615) (end 110.1 112.262792) (width 0.25) (layer "F.Cu") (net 12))
 (segment (start 111.638604 113.165) (end 110.55 112.076396) (width 0.25) (layer "F.Cu") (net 2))
 (segment (start 137.35 113.165) (end 111.638604 113.165) (width 0.25) (layer "F.Cu") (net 2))
 (segment (start 144.34 106.175) (end 137.35 113.165) (width 0.25) (layer "F.Cu") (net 2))
 (segment (start 112.657903 96.884) (end 117.697 96.884) (width 0.25) (layer "F.Cu") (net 2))
 (segment (start 110.55 112.076396) (end 110.55 98.991903) (width 0.25) (layer "F.Cu") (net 2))
 (segment (start 110.55 98.991903) (end 112.657903 96.884) (width 0.25) (layer "F.Cu") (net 2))
 (segment (start 131.75 112.715) (end 111.825 112.715) (width 0.25) (layer "F.Cu") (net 26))
 (segment (start 115.938 97.665) (end 117.697 99.424) (width 0.25) (layer "F.Cu") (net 26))
 (segment (start 111.825 112.715) (end 111 111.89) (width 0.25) (layer "F.Cu") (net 26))
 (segment (start 111 111.89) (end 111 99.178299) (width 0.25) (layer "F.Cu") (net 26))
 (segment (start 138.29 106.175) (end 131.75 112.715) (width 0.25) (layer "F.Cu") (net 26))
 (segment (start 111 99.178299) (end 112.513299 97.665) (width 0.25) (layer "F.Cu") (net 26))
 (segment (start 112.513299 97.665) (end 115.938 97.665) (width 0.25) (layer "F.Cu") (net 26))
 (segment (start 116.226 91.804) (end 117.697 91.804) (width 0.25) (layer "F.Cu") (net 22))
 (segment (start 107.5 112.25) (end 109.65 110.1) (width 0.25) (layer "F.Cu") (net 22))
 (segment (start 109.65 98.38) (end 116.226 91.804) (width 0.25) (layer "F.Cu") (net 22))
 (segment (start 103.5 112.25) (end 107.5 112.25) (width 0.25) (layer "F.Cu") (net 22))
 (segment (start 109.65 110.1) (end 109.65 98.38) (width 0.25) (layer "F.Cu") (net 22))
 (segment (start 127.14 108.35) (end 127.14 79.821) (width 0.25) (layer "B.Cu") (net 35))
 (segment (start 127.14 79.821) (end 132.937 74.024) (width 0.25) (layer "B.Cu") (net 35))
 (segment (start 123.09 100.5) (end 123.13 100.46) (width 0.25) (layer "B.Cu") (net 37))
 (segment (start 123.09 108.35) (end 123.09 100.5) (width 0.25) (layer "B.Cu") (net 37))
 (segment (start 123.13 98.635) (end 123.13 81.291) (width 0.25) (layer "B.Cu") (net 36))
 (segment (start 123.13 81.291) (end 132.937 71.484) (width 0.25) (layer "B.Cu") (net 36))
 (segment (start 123.09 81.331) (end 132.937 71.484) (width 0.25) (layer "B.Cu") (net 36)))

